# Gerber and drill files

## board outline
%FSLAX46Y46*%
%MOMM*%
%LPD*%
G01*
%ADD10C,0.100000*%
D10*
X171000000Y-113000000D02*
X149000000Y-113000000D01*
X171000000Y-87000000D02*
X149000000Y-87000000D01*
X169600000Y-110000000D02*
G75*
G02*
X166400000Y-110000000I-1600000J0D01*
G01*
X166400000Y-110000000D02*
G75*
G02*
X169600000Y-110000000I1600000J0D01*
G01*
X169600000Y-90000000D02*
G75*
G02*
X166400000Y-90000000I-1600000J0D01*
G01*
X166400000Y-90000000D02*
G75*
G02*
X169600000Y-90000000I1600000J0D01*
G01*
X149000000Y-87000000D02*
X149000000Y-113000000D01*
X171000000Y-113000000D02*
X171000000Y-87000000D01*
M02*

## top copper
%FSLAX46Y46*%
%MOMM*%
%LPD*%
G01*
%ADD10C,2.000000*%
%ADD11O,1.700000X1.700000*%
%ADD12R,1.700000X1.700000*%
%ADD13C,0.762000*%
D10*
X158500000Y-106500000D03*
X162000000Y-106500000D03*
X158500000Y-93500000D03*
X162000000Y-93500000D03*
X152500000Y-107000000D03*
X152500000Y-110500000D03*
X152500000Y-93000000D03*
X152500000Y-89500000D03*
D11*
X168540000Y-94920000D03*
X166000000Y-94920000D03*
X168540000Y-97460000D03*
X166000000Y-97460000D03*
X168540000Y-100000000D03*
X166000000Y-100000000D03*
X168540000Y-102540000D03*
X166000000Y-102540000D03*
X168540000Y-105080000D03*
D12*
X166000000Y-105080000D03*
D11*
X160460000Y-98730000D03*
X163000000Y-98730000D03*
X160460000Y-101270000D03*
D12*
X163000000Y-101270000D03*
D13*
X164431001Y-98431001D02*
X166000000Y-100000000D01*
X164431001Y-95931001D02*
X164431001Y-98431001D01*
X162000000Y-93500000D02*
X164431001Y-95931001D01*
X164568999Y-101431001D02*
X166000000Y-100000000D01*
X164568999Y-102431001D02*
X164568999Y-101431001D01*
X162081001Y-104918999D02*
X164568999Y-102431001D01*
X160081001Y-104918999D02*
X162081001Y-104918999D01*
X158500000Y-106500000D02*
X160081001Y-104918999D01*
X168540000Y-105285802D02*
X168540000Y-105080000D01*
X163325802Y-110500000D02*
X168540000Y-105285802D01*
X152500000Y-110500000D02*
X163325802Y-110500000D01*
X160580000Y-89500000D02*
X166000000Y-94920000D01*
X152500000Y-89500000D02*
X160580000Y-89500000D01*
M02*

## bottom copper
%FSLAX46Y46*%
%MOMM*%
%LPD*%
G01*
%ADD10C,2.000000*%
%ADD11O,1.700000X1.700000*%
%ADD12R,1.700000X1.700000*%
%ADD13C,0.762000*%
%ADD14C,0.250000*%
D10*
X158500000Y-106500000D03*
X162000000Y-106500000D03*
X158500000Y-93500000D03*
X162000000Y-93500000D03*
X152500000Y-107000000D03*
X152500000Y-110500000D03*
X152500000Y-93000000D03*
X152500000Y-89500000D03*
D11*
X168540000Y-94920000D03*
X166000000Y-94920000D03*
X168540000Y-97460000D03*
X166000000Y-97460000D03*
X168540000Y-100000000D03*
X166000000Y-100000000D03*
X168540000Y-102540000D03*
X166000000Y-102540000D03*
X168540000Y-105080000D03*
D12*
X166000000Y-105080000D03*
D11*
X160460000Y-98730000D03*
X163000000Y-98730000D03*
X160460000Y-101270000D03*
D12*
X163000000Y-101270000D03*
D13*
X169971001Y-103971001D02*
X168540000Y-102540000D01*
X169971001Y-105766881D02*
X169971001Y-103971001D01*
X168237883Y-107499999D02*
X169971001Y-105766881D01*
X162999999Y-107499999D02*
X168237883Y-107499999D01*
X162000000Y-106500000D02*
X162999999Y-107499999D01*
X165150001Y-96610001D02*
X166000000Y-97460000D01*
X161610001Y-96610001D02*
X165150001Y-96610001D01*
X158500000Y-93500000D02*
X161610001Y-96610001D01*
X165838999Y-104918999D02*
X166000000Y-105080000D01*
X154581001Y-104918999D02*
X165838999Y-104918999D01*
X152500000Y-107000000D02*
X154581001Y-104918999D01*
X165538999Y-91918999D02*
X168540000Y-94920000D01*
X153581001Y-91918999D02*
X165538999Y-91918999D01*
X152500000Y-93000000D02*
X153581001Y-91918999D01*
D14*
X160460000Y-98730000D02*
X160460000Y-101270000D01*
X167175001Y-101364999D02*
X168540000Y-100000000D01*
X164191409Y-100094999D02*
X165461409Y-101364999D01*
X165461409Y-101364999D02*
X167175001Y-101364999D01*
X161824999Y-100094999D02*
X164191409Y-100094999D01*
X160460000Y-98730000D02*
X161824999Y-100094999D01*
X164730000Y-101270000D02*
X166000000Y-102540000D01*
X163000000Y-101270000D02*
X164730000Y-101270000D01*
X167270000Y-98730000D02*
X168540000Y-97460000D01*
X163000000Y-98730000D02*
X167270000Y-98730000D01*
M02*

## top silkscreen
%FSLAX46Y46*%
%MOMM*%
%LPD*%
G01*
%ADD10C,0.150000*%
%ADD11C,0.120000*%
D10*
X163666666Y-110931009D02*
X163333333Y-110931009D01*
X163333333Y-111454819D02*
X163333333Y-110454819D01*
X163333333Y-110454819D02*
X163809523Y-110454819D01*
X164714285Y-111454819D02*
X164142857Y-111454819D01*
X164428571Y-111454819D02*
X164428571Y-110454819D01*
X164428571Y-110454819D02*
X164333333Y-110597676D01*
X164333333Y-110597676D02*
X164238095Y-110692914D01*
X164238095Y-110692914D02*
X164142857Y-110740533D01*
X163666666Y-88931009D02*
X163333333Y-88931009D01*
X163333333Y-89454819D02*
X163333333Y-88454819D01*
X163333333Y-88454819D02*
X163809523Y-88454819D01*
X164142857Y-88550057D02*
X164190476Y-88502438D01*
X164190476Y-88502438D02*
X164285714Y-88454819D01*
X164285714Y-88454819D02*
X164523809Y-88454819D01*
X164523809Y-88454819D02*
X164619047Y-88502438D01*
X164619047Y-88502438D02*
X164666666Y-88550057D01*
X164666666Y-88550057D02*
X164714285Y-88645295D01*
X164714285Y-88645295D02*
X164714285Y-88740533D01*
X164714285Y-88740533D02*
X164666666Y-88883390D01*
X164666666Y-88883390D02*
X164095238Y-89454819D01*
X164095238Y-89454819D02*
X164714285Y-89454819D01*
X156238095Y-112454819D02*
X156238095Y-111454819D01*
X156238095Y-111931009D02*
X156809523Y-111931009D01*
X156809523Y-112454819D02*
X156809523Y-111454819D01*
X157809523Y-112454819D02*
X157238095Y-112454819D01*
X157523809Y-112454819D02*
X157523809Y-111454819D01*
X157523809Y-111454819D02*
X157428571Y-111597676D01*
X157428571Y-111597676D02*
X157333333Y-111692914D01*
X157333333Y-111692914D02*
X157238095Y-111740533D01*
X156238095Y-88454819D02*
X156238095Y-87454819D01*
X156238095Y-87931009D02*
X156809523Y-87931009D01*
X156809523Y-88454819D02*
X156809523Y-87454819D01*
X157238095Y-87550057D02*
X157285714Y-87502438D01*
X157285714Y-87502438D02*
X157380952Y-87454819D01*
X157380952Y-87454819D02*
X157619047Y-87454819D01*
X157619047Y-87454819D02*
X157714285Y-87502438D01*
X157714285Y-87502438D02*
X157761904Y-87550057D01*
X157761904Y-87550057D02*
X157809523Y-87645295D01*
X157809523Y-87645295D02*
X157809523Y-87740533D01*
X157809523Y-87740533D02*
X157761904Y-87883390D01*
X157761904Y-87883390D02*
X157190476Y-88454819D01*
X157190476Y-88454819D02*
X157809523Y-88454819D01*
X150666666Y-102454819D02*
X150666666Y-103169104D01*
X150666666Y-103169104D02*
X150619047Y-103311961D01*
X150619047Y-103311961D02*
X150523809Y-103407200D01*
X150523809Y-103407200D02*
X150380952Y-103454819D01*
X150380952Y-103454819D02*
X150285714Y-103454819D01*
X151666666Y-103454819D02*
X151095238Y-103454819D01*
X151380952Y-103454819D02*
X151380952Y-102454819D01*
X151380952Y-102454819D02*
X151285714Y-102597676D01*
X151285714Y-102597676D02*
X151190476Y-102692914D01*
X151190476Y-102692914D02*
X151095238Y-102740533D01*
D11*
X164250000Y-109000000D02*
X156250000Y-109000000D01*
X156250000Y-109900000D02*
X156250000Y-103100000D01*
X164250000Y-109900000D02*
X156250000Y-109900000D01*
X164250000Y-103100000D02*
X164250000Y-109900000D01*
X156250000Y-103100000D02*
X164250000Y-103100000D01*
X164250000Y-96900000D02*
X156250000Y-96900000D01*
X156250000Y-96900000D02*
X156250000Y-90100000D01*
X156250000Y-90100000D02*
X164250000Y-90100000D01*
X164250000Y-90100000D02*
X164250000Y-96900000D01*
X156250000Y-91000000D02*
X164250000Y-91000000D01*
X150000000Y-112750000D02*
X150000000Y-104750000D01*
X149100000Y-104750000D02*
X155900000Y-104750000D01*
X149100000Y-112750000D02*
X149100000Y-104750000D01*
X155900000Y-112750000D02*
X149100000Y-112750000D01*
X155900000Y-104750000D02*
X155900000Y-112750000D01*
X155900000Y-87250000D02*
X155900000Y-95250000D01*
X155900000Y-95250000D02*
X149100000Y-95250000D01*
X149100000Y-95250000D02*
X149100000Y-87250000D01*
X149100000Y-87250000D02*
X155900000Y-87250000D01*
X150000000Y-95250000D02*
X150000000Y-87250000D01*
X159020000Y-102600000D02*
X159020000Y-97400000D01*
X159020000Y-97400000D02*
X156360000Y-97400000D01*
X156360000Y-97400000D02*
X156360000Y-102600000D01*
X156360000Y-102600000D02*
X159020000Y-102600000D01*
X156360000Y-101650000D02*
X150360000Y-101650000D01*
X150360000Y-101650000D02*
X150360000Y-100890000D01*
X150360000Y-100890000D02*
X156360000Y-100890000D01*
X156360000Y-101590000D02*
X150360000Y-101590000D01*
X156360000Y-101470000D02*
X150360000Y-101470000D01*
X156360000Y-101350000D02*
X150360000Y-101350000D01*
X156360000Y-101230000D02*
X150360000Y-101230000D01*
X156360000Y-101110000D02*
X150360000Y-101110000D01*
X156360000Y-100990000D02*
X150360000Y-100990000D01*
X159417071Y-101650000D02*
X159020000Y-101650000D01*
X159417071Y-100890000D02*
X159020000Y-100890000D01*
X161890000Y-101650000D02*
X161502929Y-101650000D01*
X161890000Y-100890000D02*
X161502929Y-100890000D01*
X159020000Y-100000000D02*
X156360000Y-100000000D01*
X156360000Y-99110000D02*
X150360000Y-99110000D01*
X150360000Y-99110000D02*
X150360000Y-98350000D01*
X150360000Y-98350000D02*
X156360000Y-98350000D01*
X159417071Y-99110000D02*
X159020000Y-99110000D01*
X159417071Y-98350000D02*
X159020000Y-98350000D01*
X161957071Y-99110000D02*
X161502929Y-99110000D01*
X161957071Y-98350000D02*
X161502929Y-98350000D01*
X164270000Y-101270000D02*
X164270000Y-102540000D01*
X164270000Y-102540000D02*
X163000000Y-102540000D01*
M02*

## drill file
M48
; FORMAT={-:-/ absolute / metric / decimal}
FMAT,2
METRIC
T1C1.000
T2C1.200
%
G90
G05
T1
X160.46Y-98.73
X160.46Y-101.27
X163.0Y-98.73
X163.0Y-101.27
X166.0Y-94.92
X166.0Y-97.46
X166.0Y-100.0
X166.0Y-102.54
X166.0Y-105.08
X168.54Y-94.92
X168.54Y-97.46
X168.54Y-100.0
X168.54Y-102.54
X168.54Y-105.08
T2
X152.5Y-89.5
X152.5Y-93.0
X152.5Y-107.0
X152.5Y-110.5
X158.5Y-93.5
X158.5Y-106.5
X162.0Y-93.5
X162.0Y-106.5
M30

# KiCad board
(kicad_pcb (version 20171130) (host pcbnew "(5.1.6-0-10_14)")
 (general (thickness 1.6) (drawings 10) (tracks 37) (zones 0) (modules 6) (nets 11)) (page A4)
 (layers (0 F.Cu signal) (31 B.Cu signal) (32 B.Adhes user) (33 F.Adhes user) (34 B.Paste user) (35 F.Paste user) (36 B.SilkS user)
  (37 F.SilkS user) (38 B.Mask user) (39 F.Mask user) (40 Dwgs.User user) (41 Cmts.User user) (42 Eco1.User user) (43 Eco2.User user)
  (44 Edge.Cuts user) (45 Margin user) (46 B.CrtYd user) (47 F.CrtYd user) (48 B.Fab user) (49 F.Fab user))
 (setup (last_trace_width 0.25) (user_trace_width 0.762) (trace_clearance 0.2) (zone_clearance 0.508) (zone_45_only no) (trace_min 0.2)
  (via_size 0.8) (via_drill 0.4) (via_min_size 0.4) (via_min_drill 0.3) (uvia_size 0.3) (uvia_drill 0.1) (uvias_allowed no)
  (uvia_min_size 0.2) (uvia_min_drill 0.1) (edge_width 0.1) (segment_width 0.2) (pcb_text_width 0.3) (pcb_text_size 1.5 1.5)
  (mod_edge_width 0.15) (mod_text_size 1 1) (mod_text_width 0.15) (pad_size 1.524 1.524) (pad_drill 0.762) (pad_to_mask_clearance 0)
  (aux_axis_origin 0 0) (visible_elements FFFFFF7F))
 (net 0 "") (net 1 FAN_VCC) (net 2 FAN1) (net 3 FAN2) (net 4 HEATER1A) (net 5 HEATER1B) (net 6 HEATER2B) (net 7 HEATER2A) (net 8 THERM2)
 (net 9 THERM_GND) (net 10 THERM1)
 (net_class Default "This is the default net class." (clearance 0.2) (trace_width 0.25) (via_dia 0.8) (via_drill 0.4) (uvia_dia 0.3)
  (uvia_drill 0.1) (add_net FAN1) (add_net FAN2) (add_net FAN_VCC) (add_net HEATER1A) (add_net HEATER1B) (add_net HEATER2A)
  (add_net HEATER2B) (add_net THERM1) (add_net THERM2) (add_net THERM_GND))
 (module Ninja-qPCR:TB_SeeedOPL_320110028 (layer F.Cu) (at 158.5 106.5)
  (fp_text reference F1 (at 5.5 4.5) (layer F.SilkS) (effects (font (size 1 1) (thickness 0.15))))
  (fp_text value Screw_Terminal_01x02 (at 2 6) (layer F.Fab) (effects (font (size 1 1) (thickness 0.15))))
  (fp_line (start 5.75 2.5) (end -2.25 2.5) (layer F.SilkS) (width 0.12))
  (fp_line (start -2.25 3.4) (end -2.25 -3.4) (layer F.SilkS) (width 0.12))
  (fp_line (start 5.75 3.4) (end -2.25 3.4) (layer F.SilkS) (width 0.12))
  (fp_line (start 5.75 -3.4) (end 5.75 3.4) (layer F.SilkS) (width 0.12))
  (fp_line (start -2.25 -3.4) (end 5.75 -3.4) (layer F.SilkS) (width 0.12))
  (pad 1 thru_hole circle (at 0 0) (size 2 2) (drill 1.2) (layers *.Cu *.Mask) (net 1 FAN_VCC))
  (pad 2 thru_hole circle (at 3.5 0) (size 2 2) (drill 1.2) (layers *.Cu *.Mask) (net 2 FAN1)))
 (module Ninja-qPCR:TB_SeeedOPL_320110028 (layer F.Cu) (at 162 93.5 180)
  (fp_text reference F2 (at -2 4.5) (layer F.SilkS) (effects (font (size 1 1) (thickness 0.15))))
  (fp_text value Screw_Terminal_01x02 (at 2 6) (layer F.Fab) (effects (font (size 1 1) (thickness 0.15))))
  (fp_line (start -2.25 -3.4) (end 5.75 -3.4) (layer F.SilkS) (width 0.12))
  (fp_line (start 5.75 -3.4) (end 5.75 3.4) (layer F.SilkS) (width 0.12))
  (fp_line (start 5.75 3.4) (end -2.25 3.4) (layer F.SilkS) (width 0.12))
  (fp_line (start -2.25 3.4) (end -2.25 -3.4) (layer F.SilkS) (width 0.12))
  (fp_line (start 5.75 2.5) (end -2.25 2.5) (layer F.SilkS) (width 0.12))
  (pad 2 thru_hole circle (at 3.5 0 180) (size 2 2) (drill 1.2) (layers *.Cu *.Mask) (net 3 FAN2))
  (pad 1 thru_hole circle (at 0 0 180) (size 2 2) (drill 1.2) (layers *.Cu *.Mask) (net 1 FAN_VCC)))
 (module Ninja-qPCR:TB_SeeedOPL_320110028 (layer F.Cu) (at 152.5 107 270)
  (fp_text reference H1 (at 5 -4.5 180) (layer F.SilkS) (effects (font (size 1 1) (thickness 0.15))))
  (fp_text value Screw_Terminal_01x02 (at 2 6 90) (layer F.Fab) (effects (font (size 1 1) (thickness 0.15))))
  (fp_line (start 5.75 2.5) (end -2.25 2.5) (layer F.SilkS) (width 0.12))
  (fp_line (start -2.25 3.4) (end -2.25 -3.4) (layer F.SilkS) (width 0.12))
  (fp_line (start 5.75 3.4) (end -2.25 3.4) (layer F.SilkS) (width 0.12))
  (fp_line (start 5.75 -3.4) (end 5.75 3.4) (layer F.SilkS) (width 0.12))
  (fp_line (start -2.25 -3.4) (end 5.75 -3.4) (layer F.SilkS) (width 0.12))
  (pad 1 thru_hole circle (at 0 0 270) (size 2 2) (drill 1.2) (layers *.Cu *.Mask) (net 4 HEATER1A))
  (pad 2 thru_hole circle (at 3.5 0 270) (size 2 2) (drill 1.2) (layers *.Cu *.Mask) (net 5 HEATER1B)))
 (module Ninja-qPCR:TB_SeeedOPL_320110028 (layer F.Cu) (at 152.5 89.5 270)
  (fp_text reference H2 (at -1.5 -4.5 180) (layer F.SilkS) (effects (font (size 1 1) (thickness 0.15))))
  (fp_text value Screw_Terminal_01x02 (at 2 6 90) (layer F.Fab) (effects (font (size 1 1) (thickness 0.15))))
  (fp_line (start -2.25 -3.4) (end 5.75 -3.4) (layer F.SilkS) (width 0.12))
  (fp_line (start 5.75 -3.4) (end 5.75 3.4) (layer F.SilkS) (width 0.12))
  (fp_line (start 5.75 3.4) (end -2.25 3.4) (layer F.SilkS) (width 0.12))
  (fp_line (start -2.25 3.4) (end -2.25 -3.4) (layer F.SilkS) (width 0.12))
  (fp_line (start 5.75 2.5) (end -2.25 2.5) (layer F.SilkS) (width 0.12))
  (pad 2 thru_hole circle (at 3.5 0 270) (size 2 2) (drill 1.2) (layers *.Cu *.Mask) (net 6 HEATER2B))
  (pad 1 thru_hole circle (at 0 0 270) (size 2 2) (drill 1.2) (layers *.Cu *.Mask) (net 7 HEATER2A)))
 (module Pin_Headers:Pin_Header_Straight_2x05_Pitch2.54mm (layer B.Cu) (at 166 105.08)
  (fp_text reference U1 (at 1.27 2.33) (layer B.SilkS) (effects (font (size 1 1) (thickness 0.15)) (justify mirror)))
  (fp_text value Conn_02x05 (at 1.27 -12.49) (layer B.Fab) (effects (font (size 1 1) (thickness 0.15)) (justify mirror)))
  (pad 10 thru_hole oval (at 2.54 -10.16) (size 1.7 1.7) (drill 1) (layers *.Cu *.Mask) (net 6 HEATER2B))
  (pad 9 thru_hole oval (at 0 -10.16) (size 1.7 1.7) (drill 1) (layers *.Cu *.Mask) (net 7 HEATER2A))
  (pad 8 thru_hole oval (at 2.54 -7.62) (size 1.7 1.7) (drill 1) (layers *.Cu *.Mask) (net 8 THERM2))
  (pad 7 thru_hole oval (at 0 -7.62) (size 1.7 1.7) (drill 1) (layers *.Cu *.Mask) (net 3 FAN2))
  (pad 6 thru_hole oval (at 2.54 -5.08) (size 1.7 1.7) (drill 1) (layers *.Cu *.Mask) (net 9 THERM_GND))
  (pad 5 thru_hole oval (at 0 -5.08) (size 1.7 1.7) (drill 1) (layers *.Cu *.Mask) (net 1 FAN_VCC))
  (pad 4 thru_hole oval (at 2.54 -2.54) (size 1.7 1.7) (drill 1) (layers *.Cu *.Mask) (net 2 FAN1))
  (pad 3 thru_hole oval (at 0 -2.54) (size 1.7 1.7) (drill 1) (layers *.Cu *.Mask) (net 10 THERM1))
  (pad 2 thru_hole oval (at 2.54 0) (size 1.7 1.7) (drill 1) (layers *.Cu *.Mask) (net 5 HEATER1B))
  (pad 1 thru_hole rect (at 0 0) (size 1.7 1.7) (drill 1) (layers *.Cu *.Mask) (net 4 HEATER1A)))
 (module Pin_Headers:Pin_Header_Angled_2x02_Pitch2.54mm (layer F.Cu) (at 163 101.27 180)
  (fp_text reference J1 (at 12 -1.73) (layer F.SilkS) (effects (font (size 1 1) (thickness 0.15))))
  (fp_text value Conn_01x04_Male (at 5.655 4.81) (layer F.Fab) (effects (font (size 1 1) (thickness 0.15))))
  (fp_line (start 3.98 -1.33) (end 3.98 3.87) (layer F.SilkS) (width 0.12))
  (fp_line (start 3.98 3.87) (end 6.64 3.87) (layer F.SilkS) (width 0.12))
  (fp_line (start 6.64 3.87) (end 6.64 -1.33) (layer F.SilkS) (width 0.12))
  (fp_line (start 6.64 -1.33) (end 3.98 -1.33) (layer F.SilkS) (width 0.12))
  (fp_line (start 6.64 -0.38) (end 12.64 -0.38) (layer F.SilkS) (width 0.12))
  (fp_line (start 12.64 -0.38) (end 12.64 0.38) (layer F.SilkS) (width 0.12))
  (fp_line (start 12.64 0.38) (end 6.64 0.38) (layer F.SilkS) (width 0.12))
  (fp_line (start 6.64 -0.32) (end 12.64 -0.32) (layer F.SilkS) (width 0.12))
  (fp_line (start 6.64 -0.2) (end 12.64 -0.2) (layer F.SilkS) (width 0.12))
  (fp_line (start 6.64 -0.08) (end 12.64 -0.08) (layer F.SilkS) (width 0.12))
  (fp_line (start 6.64 0.04) (end 12.64 0.04) (layer F.SilkS) (width 0.12))
  (fp_line (start 6.64 0.16) (end 12.64 0.16) (layer F.SilkS) (width 0.12))
  (fp_line (start 6.64 0.28) (end 12.64 0.28) (layer F.SilkS) (width 0.12))
  (fp_line (start 3.582929 -0.38) (end 3.98 -0.38) (layer F.SilkS) (width 0.12))
  (fp_line (start 3.582929 0.38) (end 3.98 0.38) (layer F.SilkS) (width 0.12))
  (fp_line (start 1.11 -0.38) (end 1.497071 -0.38) (layer F.SilkS) (width 0.12))
  (fp_line (start 1.11 0.38) (end 1.497071 0.38) (layer F.SilkS) (width 0.12))
  (fp_line (start 3.98 1.27) (end 6.64 1.27) (layer F.SilkS) (width 0.12))
  (fp_line (start 6.64 2.16) (end 12.64 2.16) (layer F.SilkS) (width 0.12))
  (fp_line (start 12.64 2.16) (end 12.64 2.92) (layer F.SilkS) (width 0.12))
  (fp_line (start 12.64 2.92) (end 6.64 2.92) (layer F.SilkS) (width 0.12))
  (fp_line (start 3.582929 2.16) (end 3.98 2.16) (layer F.SilkS) (width 0.12))
  (fp_line (start 3.582929 2.92) (end 3.98 2.92) (layer F.SilkS) (width 0.12))
  (fp_line (start 1.042929 2.16) (end 1.497071 2.16) (layer F.SilkS) (width 0.12))
  (fp_line (start 1.042929 2.92) (end 1.497071 2.92) (layer F.SilkS) (width 0.12))
  (fp_line (start -1.27 0) (end -1.27 -1.27) (layer F.SilkS) (width 0.12))
  (fp_line (start -1.27 -1.27) (end 0 -1.27) (layer F.SilkS) (width 0.12))
  (pad 4 thru_hole oval (at 2.54 2.54 180) (size 1.7 1.7) (drill 1) (layers *.Cu *.Mask) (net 9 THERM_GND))
  (pad 3 thru_hole oval (at 0 2.54 180) (size 1.7 1.7) (drill 1) (layers *.Cu *.Mask) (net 8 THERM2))
  (pad 2 thru_hole oval (at 2.54 0 180) (size 1.7 1.7) (drill 1) (layers *.Cu *.Mask) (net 9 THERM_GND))
  (pad 1 thru_hole rect (at 0 0 180) (size 1.7 1.7) (drill 1) (layers *.Cu *.Mask) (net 10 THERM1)))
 (gr_line (start 171 113) (end 149 113) (layer Edge.Cuts) (width 0.1))
 (gr_line (start 171 87) (end 149 87) (layer Edge.Cuts) (width 0.1))
 (gr_circle (center 168 110) (end 169.6 110) (layer Edge.Cuts) (width 0.1))
 (gr_circle (center 168 90) (end 169.6 90) (layer Edge.Cuts) (width 0.1))
 (gr_line (start 149 87) (end 149 113) (layer Edge.Cuts) (width 0.1))
 (gr_line (start 171 113) (end 171 87) (layer Edge.Cuts) (width 0.1))
 (segment (start 164.431001 98.431001) (end 166 100) (width 0.762) (layer F.Cu) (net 1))
 (segment (start 164.431001 95.931001) (end 164.431001 98.431001) (width 0.762) (layer F.Cu) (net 1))
 (segment (start 162 93.5) (end 164.431001 95.931001) (width 0.762) (layer F.Cu) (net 1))
 (segment (start 164.568999 101.431001) (end 166 100) (width 0.762) (layer F.Cu) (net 1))
 (segment (start 164.568999 102.431001) (end 164.568999 101.431001) (width 0.762) (layer F.Cu) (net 1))
 (segment (start 162.081001 104.918999) (end 164.568999 102.431001) (width 0.762) (layer F.Cu) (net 1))
 (segment (start 160.081001 104.918999) (end 162.081001 104.918999) (width 0.762) (layer F.Cu) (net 1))
 (segment (start 158.5 106.5) (end 160.081001 104.918999) (width 0.762) (layer F.Cu) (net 1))
 (segment (start 169.971001 103.971001) (end 168.54 102.54) (width 0.762) (layer B.Cu) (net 2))
 (segment (start 169.971001 105.766881) (end 169.971001 103.971001) (width 0.762) (layer B.Cu) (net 2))
 (segment (start 168.237883 107.499999) (end 169.971001 105.766881) (width 0.762) (layer B.Cu) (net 2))
 (segment (start 162.999999 107.499999) (end 168.237883 107.499999) (width 0.762) (layer B.Cu) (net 2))
 (segment (start 162 106.5) (end 162.999999 107.499999) (width 0.762) (layer B.Cu) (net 2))
 (segment (start 165.150001 96.610001) (end 166 97.46) (width 0.762) (layer B.Cu) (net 3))
 (segment (start 161.610001 96.610001) (end 165.150001 96.610001) (width 0.762) (layer B.Cu) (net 3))
 (segment (start 158.5 93.5) (end 161.610001 96.610001) (width 0.762) (layer B.Cu) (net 3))
 (segment (start 165.838999 104.918999) (end 166 105.08) (width 0.762) (layer B.Cu) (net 4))
 (segment (start 154.581001 104.918999) (end 165.838999 104.918999) (width 0.762) (layer B.Cu) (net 4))
 (segment (start 152.5 107) (end 154.581001 104.918999) (width 0.762) (layer B.Cu) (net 4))
 (segment (start 168.54 105.285802) (end 168.54 105.08) (width 0.762) (layer F.Cu) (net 5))
 (segment (start 163.325802 110.5) (end 168.54 105.285802) (width 0.762) (layer F.Cu) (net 5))
 (segment (start 152.5 110.5) (end 163.325802 110.5) (width 0.762) (layer F.Cu) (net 5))
 (segment (start 165.538999 91.918999) (end 168.54 94.92) (width 0.762) (layer B.Cu) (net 6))
 (segment (start 153.581001 91.918999) (end 165.538999 91.918999) (width 0.762) (layer B.Cu) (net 6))
 (segment (start 152.5 93) (end 153.581001 91.918999) (width 0.762) (layer B.Cu) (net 6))
 (segment (start 160.58 89.5) (end 166 94.92) (width 0.762) (layer F.Cu) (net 7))
 (segment (start 152.5 89.5) (end 160.58 89.5) (width 0.762) (layer F.Cu) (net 7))
 (segment (start 160.46 98.73) (end 160.46 101.27) (width 0.25) (layer B.Cu) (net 9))
 (segment (start 167.175001 101.364999) (end 168.54 100) (width 0.25) (layer B.Cu) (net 9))
 (segment (start 164.191409 100.094999) (end 165.461409 101.364999) (width 0.25) (layer B.Cu) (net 9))
 (segment (start 165.461409 101.364999) (end 167.175001 101.364999) (width 0.25) (layer B.Cu) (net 9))
 (segment (start 161.824999 100.094999) (end 164.191409 100.094999) (width 0.25) (layer B.Cu) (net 9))
 (segment (start 160.46 98.73) (end 161.824999 100.094999) (width 0.25) (layer B.Cu) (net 9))
 (segment (start 164.73 101.27) (end 166 102.54) (width 0.25) (layer B.Cu) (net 10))
 (segment (start 163 101.27) (end 164.73 101.27) (width 0.25) (layer B.Cu) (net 10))
 (segment (start 167.27 98.73) (end 168.54 97.46) (width 0.25) (layer B.Cu) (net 8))
 (segment (start 163 98.73) (end 167.27 98.73) (width 0.25) (layer B.Cu) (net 8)))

